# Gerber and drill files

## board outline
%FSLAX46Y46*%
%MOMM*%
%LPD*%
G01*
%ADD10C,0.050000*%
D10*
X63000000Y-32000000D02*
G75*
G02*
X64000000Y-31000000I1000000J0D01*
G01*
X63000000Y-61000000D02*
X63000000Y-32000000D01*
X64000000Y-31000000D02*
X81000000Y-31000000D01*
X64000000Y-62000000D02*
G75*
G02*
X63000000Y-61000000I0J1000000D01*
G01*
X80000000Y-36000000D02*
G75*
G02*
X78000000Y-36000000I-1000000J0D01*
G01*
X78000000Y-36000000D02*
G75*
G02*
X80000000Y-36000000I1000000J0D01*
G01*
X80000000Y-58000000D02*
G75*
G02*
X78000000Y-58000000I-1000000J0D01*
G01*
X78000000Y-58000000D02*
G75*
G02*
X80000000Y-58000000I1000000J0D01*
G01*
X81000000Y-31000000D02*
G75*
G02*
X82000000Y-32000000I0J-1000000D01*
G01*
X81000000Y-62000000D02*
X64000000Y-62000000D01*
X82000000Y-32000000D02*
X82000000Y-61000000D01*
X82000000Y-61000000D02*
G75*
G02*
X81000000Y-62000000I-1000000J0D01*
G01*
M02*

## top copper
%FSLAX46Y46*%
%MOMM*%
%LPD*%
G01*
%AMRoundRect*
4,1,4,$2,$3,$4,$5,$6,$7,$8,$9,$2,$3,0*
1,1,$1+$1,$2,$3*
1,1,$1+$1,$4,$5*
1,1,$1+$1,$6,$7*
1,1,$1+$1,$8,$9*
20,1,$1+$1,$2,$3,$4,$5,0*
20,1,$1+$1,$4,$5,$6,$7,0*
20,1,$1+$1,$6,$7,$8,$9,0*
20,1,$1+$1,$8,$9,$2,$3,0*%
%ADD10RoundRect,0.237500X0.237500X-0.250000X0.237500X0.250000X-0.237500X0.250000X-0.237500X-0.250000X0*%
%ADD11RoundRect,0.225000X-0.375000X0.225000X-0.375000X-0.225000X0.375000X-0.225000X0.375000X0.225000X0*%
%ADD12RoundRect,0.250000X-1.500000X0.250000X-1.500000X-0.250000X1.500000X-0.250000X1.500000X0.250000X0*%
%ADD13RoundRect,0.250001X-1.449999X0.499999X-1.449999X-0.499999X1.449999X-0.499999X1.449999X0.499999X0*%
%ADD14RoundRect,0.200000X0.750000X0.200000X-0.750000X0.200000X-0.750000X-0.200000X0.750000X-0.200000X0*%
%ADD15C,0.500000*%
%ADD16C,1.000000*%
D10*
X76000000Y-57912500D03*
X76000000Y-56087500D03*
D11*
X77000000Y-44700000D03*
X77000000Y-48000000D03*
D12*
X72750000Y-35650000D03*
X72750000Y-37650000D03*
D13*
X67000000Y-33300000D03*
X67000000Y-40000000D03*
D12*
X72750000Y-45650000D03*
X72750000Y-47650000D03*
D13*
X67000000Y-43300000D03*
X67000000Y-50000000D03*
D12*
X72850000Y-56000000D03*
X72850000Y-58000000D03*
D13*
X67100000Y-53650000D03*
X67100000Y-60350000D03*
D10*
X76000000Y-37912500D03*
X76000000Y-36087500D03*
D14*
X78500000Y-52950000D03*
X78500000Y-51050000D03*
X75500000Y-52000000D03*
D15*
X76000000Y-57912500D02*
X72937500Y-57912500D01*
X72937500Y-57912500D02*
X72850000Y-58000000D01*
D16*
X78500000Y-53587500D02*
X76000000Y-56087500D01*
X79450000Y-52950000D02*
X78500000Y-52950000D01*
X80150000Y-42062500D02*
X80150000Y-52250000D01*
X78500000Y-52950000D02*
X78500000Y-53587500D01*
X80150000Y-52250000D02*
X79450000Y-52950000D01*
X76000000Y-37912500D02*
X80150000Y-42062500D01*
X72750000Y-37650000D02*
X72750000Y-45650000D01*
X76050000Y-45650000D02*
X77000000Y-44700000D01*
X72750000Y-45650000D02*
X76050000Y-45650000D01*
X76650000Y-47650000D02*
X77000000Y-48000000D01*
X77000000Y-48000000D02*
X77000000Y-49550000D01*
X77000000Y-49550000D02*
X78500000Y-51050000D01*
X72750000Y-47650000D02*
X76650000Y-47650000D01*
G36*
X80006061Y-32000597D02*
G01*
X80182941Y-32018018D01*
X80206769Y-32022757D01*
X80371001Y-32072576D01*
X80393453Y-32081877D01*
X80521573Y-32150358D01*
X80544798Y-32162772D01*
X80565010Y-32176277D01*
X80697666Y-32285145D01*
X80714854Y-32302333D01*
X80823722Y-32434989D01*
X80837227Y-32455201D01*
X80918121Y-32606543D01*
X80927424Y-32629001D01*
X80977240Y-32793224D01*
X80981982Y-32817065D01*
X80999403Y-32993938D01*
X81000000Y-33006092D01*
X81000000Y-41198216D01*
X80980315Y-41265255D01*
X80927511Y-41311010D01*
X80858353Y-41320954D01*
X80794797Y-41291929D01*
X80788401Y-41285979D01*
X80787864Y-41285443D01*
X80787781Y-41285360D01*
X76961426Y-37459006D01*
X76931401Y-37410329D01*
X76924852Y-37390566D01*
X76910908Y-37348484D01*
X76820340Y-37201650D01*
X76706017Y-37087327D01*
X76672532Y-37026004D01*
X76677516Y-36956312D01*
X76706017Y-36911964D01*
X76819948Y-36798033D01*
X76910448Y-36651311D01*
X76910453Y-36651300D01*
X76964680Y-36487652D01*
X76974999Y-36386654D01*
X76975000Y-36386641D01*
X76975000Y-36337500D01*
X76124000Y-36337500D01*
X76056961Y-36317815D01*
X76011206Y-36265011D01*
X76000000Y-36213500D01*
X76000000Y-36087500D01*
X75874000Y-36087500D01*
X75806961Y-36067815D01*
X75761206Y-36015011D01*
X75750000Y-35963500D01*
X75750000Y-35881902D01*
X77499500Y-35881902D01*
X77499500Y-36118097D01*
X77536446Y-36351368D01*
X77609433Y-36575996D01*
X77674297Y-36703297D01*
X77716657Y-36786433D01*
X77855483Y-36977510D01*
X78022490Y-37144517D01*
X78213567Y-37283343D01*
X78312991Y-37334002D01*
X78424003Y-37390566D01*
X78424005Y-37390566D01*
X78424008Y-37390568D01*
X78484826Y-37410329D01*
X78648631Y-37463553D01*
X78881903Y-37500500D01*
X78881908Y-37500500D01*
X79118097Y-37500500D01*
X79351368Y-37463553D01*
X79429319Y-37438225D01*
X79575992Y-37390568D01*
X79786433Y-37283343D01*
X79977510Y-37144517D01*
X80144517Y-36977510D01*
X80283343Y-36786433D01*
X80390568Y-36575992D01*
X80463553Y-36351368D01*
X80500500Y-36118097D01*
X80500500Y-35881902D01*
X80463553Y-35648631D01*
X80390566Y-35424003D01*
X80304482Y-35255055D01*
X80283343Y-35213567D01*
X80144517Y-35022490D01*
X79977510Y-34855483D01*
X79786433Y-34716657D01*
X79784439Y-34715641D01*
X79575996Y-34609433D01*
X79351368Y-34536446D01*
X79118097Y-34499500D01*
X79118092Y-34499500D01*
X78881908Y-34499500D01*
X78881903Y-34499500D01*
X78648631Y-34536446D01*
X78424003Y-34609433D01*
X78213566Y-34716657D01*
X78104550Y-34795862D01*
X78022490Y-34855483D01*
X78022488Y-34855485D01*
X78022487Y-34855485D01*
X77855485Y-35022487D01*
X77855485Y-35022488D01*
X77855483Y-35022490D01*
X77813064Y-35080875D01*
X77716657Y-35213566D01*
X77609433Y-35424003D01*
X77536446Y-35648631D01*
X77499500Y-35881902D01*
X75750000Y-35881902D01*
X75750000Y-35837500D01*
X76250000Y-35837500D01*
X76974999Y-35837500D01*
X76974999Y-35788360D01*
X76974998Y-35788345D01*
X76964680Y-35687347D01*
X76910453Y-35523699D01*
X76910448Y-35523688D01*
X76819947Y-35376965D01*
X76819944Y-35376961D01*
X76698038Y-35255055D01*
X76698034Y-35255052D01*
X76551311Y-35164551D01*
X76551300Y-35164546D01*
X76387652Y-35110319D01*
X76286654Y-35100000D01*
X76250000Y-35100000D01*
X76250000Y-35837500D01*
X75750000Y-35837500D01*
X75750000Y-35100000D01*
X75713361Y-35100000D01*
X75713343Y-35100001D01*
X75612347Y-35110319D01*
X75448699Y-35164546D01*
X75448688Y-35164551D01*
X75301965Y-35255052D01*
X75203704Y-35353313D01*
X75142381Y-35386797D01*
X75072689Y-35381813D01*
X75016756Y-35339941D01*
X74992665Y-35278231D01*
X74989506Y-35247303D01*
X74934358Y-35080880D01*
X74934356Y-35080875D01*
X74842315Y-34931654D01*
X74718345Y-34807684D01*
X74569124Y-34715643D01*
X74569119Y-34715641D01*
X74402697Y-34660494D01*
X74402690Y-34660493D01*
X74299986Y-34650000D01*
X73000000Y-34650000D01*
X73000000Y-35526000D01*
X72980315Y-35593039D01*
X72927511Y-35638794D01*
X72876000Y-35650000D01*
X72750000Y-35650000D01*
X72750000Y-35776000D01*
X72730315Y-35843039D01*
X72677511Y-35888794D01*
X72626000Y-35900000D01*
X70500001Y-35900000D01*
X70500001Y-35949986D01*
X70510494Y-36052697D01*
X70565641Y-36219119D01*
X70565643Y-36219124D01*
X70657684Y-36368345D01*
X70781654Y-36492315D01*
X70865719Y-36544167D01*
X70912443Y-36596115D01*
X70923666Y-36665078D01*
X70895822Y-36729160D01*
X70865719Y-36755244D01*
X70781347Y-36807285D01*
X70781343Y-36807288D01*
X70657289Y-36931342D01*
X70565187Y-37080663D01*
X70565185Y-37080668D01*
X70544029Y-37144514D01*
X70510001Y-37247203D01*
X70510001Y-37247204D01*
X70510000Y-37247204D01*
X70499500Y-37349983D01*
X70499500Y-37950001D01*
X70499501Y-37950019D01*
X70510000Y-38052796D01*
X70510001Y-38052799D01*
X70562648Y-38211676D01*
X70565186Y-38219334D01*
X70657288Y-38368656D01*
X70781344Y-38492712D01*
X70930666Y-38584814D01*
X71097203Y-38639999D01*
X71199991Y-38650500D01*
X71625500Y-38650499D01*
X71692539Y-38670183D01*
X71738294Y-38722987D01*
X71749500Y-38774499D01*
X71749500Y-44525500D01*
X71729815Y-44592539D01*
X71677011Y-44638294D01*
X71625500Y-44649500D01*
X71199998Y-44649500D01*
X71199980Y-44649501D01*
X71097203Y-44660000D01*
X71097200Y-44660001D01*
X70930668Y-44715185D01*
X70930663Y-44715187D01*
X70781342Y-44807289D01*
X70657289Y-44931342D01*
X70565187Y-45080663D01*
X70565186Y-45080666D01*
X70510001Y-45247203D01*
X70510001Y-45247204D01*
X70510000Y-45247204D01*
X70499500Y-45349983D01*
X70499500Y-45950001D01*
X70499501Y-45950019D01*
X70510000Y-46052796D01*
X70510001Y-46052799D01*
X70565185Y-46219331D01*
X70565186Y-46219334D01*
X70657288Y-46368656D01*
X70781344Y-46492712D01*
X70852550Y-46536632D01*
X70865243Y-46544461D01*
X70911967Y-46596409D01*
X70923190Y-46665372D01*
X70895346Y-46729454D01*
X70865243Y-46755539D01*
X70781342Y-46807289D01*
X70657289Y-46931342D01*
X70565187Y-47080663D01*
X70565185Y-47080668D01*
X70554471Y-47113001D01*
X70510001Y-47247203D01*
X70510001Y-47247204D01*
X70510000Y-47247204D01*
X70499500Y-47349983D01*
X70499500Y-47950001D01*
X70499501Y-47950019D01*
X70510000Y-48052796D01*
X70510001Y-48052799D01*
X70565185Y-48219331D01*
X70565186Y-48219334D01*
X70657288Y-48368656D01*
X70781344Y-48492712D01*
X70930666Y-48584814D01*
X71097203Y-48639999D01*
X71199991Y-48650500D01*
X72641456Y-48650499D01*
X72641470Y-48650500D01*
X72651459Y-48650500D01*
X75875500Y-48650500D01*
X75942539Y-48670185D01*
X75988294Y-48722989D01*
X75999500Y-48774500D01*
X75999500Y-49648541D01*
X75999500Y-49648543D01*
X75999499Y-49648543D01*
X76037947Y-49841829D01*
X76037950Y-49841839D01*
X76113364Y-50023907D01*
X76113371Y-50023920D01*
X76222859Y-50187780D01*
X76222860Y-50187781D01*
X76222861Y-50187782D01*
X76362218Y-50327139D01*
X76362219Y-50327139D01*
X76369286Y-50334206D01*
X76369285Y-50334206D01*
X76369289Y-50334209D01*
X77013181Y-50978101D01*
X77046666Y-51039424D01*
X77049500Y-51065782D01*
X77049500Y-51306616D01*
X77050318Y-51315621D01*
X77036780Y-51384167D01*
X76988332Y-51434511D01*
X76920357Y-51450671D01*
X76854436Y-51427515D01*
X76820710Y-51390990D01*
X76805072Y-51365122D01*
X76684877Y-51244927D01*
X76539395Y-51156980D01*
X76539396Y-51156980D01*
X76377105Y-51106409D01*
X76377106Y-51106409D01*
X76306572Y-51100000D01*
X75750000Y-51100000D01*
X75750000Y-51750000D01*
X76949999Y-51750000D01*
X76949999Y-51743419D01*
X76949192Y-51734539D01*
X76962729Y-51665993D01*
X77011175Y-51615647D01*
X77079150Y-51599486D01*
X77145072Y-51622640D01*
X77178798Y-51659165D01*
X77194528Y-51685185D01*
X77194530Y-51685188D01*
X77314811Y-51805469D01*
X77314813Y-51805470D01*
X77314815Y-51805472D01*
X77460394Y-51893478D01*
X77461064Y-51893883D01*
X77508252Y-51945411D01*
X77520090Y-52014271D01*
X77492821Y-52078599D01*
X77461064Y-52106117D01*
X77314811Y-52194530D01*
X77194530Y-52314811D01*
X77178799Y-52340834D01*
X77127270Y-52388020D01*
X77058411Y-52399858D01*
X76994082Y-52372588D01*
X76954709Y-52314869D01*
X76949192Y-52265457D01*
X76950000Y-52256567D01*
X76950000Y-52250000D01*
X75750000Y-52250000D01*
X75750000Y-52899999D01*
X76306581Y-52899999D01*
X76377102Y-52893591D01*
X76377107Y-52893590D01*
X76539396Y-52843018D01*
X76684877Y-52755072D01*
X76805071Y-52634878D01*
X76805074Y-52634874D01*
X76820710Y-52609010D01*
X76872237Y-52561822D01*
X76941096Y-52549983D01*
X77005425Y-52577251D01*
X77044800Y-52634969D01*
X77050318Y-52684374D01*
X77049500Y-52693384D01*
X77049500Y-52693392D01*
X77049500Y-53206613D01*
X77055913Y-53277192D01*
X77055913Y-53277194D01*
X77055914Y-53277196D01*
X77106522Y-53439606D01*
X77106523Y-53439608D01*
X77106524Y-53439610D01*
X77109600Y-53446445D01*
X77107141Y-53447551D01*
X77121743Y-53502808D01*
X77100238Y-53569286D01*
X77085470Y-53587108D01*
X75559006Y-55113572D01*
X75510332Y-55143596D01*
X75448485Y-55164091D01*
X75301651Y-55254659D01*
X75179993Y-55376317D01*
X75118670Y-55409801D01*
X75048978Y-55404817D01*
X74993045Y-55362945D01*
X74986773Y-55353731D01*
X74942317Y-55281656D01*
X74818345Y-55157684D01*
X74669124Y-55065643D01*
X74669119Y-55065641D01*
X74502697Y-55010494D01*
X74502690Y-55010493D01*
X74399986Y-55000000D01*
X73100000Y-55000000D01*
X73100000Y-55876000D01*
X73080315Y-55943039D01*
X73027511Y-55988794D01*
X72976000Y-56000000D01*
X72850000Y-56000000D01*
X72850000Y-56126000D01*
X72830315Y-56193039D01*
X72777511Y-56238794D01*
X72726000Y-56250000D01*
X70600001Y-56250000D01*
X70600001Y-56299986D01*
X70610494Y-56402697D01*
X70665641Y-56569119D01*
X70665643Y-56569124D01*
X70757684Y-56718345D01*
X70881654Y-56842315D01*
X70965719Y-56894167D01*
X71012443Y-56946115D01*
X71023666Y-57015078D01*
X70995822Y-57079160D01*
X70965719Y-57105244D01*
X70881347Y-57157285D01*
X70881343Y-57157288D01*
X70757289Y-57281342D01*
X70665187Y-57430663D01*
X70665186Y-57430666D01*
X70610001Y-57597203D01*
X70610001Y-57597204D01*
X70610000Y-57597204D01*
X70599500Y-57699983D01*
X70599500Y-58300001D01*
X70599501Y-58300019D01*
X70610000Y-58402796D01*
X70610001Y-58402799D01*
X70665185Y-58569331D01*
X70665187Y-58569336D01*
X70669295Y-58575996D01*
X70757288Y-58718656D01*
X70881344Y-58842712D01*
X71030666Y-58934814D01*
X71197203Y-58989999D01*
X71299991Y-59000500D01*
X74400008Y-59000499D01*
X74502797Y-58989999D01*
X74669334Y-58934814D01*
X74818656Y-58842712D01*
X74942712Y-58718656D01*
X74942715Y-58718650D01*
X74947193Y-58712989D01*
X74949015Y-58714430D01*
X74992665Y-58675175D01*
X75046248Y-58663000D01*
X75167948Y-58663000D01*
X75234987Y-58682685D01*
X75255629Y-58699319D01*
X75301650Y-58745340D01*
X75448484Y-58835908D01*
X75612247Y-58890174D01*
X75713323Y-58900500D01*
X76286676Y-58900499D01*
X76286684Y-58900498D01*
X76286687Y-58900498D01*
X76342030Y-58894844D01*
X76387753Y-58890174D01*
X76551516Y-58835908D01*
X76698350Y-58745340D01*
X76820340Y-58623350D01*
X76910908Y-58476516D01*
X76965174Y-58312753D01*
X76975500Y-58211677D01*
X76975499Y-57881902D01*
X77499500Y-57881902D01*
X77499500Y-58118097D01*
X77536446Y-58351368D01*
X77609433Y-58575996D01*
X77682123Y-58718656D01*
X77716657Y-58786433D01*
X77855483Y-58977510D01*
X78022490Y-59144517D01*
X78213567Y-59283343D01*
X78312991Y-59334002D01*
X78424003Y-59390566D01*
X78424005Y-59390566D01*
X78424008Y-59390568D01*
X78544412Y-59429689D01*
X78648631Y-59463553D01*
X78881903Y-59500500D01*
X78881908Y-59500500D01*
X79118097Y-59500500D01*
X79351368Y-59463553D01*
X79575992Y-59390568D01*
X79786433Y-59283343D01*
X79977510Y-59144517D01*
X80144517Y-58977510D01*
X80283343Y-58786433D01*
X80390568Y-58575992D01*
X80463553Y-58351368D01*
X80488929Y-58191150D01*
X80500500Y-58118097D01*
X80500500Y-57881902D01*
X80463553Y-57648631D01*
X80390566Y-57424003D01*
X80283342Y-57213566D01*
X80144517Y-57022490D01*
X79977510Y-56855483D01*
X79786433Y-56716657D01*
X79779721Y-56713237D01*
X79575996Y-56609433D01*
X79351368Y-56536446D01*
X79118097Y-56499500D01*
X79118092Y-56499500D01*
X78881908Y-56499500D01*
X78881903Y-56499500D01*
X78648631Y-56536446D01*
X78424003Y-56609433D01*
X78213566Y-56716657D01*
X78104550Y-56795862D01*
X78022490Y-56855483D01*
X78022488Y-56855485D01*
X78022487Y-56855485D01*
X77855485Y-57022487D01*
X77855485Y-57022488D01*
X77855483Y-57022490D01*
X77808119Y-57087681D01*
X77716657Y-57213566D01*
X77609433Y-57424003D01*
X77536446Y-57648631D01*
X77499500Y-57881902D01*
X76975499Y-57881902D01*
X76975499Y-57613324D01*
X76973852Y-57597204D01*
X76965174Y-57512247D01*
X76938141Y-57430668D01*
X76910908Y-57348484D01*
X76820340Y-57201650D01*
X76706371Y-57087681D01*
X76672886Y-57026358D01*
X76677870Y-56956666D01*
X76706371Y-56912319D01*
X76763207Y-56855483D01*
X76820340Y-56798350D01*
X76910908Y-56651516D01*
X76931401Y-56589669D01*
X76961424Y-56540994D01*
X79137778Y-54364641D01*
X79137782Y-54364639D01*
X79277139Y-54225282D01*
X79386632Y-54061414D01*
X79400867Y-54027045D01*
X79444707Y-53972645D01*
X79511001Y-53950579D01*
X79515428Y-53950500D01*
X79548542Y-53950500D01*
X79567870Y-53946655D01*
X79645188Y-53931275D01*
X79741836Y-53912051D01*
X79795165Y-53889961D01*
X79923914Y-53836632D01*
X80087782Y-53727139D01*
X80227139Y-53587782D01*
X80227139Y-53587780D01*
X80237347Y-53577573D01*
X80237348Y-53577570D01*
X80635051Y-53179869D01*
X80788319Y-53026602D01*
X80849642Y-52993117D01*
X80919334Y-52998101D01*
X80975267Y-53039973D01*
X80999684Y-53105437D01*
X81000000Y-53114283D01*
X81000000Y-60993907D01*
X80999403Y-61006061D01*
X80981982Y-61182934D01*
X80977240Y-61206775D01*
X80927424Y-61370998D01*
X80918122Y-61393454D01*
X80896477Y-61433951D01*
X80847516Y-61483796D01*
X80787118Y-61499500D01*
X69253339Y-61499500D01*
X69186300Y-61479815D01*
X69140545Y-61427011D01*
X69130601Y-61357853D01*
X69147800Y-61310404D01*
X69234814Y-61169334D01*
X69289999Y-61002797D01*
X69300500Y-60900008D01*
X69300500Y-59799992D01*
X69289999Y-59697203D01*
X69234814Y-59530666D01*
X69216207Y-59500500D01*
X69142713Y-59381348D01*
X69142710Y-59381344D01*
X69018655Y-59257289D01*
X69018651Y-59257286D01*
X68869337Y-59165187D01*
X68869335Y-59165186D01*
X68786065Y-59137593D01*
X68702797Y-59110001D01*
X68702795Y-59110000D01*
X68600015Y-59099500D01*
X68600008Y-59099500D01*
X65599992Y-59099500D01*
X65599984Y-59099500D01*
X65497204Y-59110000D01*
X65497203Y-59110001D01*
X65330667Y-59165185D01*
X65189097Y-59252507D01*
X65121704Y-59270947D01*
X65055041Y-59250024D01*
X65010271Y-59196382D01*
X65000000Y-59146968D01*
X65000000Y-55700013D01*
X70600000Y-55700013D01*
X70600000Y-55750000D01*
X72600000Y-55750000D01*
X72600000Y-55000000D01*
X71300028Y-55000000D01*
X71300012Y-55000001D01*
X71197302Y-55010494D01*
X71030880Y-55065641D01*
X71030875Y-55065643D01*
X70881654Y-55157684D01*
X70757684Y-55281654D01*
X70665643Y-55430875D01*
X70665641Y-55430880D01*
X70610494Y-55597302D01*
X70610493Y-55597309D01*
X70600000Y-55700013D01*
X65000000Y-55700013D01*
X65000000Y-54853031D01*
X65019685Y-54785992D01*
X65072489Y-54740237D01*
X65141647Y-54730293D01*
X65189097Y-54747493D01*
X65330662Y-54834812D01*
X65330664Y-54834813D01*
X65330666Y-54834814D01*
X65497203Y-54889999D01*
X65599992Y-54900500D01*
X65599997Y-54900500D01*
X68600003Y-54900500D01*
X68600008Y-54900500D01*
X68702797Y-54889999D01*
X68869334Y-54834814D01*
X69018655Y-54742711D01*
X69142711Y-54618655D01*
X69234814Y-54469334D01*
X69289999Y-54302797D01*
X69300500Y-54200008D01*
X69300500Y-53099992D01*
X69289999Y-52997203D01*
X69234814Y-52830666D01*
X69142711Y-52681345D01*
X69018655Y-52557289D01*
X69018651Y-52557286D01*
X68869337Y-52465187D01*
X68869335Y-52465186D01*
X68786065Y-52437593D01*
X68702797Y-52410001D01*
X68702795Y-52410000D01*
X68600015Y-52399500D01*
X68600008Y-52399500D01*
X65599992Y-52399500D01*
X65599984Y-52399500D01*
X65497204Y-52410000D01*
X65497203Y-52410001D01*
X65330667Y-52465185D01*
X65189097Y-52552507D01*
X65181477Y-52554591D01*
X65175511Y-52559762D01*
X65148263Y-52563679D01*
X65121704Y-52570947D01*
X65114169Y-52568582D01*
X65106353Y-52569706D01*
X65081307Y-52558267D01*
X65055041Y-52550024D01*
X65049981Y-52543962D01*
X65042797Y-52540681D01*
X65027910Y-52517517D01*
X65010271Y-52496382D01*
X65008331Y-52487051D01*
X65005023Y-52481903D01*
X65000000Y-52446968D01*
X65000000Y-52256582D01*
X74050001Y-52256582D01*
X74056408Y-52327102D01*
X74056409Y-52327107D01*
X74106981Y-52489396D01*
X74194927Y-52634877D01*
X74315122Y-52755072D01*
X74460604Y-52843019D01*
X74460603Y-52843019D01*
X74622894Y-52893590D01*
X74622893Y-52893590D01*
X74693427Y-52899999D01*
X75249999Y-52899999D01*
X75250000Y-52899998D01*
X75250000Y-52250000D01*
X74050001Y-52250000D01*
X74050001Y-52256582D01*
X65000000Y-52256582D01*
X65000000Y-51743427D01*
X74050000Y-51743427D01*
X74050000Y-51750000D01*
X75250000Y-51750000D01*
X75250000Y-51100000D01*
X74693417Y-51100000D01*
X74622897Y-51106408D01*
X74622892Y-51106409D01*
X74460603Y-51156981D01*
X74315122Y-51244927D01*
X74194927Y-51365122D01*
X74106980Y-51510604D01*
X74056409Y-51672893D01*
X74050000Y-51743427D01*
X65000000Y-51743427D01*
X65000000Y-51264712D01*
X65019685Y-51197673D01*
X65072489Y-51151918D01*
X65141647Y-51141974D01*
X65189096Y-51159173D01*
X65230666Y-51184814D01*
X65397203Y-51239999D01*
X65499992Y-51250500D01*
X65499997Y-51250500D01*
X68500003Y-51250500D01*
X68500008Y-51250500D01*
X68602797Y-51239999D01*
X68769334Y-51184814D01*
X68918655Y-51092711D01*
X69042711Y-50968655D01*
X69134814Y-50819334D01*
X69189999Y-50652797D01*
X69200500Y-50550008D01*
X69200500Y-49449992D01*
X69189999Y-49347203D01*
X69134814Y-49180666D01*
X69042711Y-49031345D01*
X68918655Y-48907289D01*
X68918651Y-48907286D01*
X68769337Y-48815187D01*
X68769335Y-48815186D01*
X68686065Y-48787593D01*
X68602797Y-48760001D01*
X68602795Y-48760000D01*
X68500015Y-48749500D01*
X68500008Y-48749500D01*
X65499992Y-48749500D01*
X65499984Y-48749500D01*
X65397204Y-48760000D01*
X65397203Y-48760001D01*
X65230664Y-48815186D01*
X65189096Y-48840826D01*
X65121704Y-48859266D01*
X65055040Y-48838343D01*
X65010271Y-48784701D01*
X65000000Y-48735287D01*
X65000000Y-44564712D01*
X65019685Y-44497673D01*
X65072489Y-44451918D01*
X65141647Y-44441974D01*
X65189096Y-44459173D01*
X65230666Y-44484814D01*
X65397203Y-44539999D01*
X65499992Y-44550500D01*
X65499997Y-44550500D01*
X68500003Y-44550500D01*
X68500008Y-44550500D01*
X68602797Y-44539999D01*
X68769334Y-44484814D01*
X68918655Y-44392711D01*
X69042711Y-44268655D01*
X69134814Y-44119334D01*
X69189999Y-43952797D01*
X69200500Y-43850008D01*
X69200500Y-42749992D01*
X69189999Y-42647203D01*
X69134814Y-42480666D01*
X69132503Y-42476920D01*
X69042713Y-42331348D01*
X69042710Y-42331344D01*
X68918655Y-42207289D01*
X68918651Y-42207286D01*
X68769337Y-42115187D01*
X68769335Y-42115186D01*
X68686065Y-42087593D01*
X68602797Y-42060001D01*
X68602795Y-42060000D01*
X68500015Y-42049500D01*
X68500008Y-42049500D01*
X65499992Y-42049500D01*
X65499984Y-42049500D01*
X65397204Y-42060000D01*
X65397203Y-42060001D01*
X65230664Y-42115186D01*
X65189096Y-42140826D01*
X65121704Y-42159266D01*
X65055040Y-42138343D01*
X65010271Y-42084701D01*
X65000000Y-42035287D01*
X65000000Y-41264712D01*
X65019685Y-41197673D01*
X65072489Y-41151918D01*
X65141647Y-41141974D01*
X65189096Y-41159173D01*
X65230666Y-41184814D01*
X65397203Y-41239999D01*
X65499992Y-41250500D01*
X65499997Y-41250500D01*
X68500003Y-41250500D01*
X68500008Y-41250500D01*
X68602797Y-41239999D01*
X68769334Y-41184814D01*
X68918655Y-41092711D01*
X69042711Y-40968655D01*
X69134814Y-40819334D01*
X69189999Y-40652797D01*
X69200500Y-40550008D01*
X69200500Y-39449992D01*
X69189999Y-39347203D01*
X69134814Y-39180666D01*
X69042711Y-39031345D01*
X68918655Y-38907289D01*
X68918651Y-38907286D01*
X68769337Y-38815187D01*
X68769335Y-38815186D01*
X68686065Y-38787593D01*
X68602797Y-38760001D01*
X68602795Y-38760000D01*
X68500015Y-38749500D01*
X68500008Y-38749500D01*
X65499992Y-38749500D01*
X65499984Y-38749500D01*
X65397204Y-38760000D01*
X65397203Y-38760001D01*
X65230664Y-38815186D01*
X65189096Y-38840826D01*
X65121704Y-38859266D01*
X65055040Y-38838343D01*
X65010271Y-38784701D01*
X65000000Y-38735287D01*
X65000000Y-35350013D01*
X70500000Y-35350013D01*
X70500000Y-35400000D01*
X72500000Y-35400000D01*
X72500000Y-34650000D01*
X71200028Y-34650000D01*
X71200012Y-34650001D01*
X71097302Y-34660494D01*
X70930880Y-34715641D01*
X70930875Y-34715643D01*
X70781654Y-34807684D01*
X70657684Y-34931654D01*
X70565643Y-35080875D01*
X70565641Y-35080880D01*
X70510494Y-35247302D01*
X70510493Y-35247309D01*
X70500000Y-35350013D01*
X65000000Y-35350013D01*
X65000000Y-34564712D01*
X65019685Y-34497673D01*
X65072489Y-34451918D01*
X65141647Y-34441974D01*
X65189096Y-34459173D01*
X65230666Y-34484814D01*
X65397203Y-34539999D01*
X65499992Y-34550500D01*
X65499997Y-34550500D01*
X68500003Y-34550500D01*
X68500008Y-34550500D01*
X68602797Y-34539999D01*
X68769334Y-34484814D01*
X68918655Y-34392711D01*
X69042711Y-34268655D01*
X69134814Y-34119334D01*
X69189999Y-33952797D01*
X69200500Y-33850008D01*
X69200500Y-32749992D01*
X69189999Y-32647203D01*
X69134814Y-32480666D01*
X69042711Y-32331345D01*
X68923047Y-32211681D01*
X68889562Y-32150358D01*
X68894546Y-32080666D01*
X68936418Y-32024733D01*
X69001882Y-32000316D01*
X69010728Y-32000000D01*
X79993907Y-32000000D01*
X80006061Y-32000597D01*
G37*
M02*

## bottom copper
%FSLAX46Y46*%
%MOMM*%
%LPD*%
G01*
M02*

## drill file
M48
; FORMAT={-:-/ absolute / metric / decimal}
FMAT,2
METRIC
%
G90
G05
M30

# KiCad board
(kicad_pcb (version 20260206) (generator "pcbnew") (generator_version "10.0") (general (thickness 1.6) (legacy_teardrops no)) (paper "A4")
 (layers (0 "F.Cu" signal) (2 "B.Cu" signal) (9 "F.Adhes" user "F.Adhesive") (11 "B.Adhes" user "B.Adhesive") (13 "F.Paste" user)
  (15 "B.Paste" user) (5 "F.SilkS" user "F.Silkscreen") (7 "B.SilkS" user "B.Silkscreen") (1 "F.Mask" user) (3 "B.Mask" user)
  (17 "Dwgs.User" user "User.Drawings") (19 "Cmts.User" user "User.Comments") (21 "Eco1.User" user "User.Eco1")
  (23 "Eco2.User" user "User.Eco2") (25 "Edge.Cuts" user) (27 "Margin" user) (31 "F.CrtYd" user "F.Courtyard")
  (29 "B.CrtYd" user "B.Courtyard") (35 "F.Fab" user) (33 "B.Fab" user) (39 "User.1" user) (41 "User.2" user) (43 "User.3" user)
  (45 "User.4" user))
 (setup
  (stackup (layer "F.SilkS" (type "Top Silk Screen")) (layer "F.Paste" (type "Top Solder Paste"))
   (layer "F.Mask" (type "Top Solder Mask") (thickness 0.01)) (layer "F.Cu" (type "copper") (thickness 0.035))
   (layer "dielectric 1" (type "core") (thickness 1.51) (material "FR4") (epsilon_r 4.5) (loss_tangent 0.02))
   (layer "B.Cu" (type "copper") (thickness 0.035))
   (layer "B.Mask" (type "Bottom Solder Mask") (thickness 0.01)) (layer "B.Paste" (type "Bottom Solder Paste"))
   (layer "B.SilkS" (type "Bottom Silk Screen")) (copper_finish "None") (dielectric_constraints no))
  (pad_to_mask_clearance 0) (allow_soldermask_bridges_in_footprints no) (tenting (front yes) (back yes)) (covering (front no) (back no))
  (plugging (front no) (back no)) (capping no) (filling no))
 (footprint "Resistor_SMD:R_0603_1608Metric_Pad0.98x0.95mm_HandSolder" (layer "F.Cu") (at 76 57 90)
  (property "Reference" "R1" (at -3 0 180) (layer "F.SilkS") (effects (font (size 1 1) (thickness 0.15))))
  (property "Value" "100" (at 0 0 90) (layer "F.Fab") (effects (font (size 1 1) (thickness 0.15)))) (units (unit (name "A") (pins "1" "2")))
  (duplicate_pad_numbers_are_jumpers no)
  (pad "1" smd roundrect (at -0.9125 0 90) (size 0.975 0.95) (layers "F.Cu" "F.Mask" "F.Paste") (roundrect_rratio 0.25)
   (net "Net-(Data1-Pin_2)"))
  (pad "2" smd roundrect (at 0.9125 0 90) (size 0.975 0.95) (layers "F.Cu" "F.Mask" "F.Paste") (roundrect_rratio 0.25) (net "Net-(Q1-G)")))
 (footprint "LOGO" (layer "F.Cu") (at 80 44 -90)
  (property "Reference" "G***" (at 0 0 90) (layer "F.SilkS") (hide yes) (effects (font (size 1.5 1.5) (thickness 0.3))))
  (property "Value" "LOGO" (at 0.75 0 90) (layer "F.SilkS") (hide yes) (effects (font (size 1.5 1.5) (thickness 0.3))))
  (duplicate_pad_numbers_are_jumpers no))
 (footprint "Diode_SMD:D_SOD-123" (layer "F.Cu") (at 77 46.35 -90)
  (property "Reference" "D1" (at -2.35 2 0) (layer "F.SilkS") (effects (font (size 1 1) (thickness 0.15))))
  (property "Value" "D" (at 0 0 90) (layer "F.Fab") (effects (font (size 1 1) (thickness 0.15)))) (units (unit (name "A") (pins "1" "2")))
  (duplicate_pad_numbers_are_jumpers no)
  (pad "1" smd roundrect (at -1.65 0 270) (size 0.9 1.2) (layers "F.Cu" "F.Mask" "F.Paste") (roundrect_rratio 0.25) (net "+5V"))
  (pad "2" smd roundrect (at 1.65 0 270) (size 0.9 1.2) (layers "F.Cu" "F.Mask" "F.Paste") (roundrect_rratio 0.25) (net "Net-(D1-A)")))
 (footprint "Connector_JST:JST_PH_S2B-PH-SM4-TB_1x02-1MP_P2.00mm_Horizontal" (layer "F.Cu") (at 69.9 36.65 -90)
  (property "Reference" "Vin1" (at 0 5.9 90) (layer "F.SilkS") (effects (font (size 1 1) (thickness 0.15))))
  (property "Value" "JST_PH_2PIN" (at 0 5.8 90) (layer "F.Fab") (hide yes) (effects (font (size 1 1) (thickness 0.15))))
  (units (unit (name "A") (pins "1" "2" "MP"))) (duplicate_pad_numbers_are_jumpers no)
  (pad "1" smd roundrect (at -1 -2.85 270) (size 1 3.5) (layers "F.Cu" "F.Mask" "F.Paste") (roundrect_rratio 0.25) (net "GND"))
  (pad "2" smd roundrect (at 1 -2.85 270) (size 1 3.5) (layers "F.Cu" "F.Mask" "F.Paste") (roundrect_rratio 0.25) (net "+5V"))
  (pad "MP" smd roundrect (at -3.35 2.9 270) (size 1.5 3.4) (layers "F.Cu" "F.Mask" "F.Paste") (roundrect_rratio 0.166667)
   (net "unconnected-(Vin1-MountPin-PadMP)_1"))
  (pad "MP" smd roundrect (at 3.35 2.9 270) (size 1.5 3.4) (layers "F.Cu" "F.Mask" "F.Paste") (roundrect_rratio 0.166667)
   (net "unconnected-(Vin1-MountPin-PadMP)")))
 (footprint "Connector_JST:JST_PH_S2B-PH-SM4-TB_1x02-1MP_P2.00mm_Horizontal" (layer "F.Cu") (at 69.9 46.65 -90)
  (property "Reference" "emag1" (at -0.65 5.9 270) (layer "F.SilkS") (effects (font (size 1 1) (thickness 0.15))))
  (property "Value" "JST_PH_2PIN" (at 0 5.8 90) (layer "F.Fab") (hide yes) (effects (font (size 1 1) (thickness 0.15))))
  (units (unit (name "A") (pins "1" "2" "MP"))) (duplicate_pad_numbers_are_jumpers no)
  (pad "1" smd roundrect (at -1 -2.85 270) (size 1 3.5) (layers "F.Cu" "F.Mask" "F.Paste") (roundrect_rratio 0.25) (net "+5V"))
  (pad "2" smd roundrect (at 1 -2.85 270) (size 1 3.5) (layers "F.Cu" "F.Mask" "F.Paste") (roundrect_rratio 0.25) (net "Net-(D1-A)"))
  (pad "MP" smd roundrect (at -3.35 2.9 270) (size 1.5 3.4) (layers "F.Cu" "F.Mask" "F.Paste") (roundrect_rratio 0.166667)
   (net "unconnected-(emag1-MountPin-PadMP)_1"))
  (pad "MP" smd roundrect (at 3.35 2.9 270) (size 1.5 3.4) (layers "F.Cu" "F.Mask" "F.Paste") (roundrect_rratio 0.166667)
   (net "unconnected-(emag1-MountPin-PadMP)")))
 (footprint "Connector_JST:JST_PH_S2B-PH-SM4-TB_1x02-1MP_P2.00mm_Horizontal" (layer "F.Cu") (at 70 57 -90)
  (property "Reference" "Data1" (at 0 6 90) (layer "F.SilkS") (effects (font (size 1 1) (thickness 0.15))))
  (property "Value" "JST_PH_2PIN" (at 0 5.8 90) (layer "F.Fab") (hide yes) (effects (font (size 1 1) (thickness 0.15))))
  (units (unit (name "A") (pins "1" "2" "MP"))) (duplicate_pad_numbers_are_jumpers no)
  (pad "1" smd roundrect (at -1 -2.85 270) (size 1 3.5) (layers "F.Cu" "F.Mask" "F.Paste") (roundrect_rratio 0.25) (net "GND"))
  (pad "2" smd roundrect (at 1 -2.85 270) (size 1 3.5) (layers "F.Cu" "F.Mask" "F.Paste") (roundrect_rratio 0.25) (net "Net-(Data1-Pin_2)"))
  (pad "MP" smd roundrect (at -3.35 2.9 270) (size 1.5 3.4) (layers "F.Cu" "F.Mask" "F.Paste") (roundrect_rratio 0.166667)
   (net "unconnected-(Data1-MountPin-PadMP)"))
  (pad "MP" smd roundrect (at 3.35 2.9 270) (size 1.5 3.4) (layers "F.Cu" "F.Mask" "F.Paste") (roundrect_rratio 0.166667)
   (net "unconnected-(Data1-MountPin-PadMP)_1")))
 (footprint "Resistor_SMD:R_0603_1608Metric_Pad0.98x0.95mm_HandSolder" (layer "F.Cu") (at 76 37 90)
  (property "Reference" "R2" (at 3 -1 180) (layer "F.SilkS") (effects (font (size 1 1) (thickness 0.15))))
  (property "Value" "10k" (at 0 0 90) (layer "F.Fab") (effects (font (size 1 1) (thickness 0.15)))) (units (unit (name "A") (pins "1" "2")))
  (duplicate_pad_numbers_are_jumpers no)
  (pad "1" smd roundrect (at -0.9125 0 90) (size 0.975 0.95) (layers "F.Cu" "F.Mask" "F.Paste") (roundrect_rratio 0.25) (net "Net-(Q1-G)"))
  (pad "2" smd roundrect (at 0.9125 0 90) (size 0.975 0.95) (layers "F.Cu" "F.Mask" "F.Paste") (roundrect_rratio 0.25) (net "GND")))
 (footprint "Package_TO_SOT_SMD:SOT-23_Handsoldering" (layer "F.Cu") (at 77 52 180)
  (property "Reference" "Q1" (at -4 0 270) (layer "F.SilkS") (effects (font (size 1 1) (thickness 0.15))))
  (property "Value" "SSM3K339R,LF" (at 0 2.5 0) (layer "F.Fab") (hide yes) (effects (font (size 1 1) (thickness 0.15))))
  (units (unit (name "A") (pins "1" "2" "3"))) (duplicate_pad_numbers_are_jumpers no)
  (pad "1" smd roundrect (at -1.5 -0.95 180) (size 1.9 0.8) (layers "F.Cu" "F.Mask" "F.Paste") (roundrect_rratio 0.25) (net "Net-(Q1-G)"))
  (pad "2" smd roundrect (at -1.5 0.95 180) (size 1.9 0.8) (layers "F.Cu" "F.Mask" "F.Paste") (roundrect_rratio 0.25) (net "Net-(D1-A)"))
  (pad "3" smd roundrect (at 1.5 0 180) (size 1.9 0.8) (layers "F.Cu" "F.Mask" "F.Paste") (roundrect_rratio 0.25) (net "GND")))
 (gr_arc (start 63 32) (mid 63.292893 31.292893) (end 64 31) (stroke (width 0.05) (type default)) (layer "Edge.Cuts"))
 (gr_line (start 63 61) (end 63 32) (stroke (width 0.05) (type default)) (layer "Edge.Cuts"))
 (gr_line (start 64 31) (end 81 31) (stroke (width 0.05) (type default)) (layer "Edge.Cuts"))
 (gr_arc (start 64 62) (mid 63.292893 61.707107) (end 63 61) (stroke (width 0.05) (type default)) (layer "Edge.Cuts"))
 (gr_circle (center 79 36) (end 79 37) (stroke (width 0.05) (type default)) (fill no) (layer "Edge.Cuts"))
 (gr_circle (center 79 58) (end 79 59) (stroke (width 0.05) (type default)) (fill no) (layer "Edge.Cuts"))
 (gr_arc (start 81 31) (mid 81.707107 31.292893) (end 82 32) (stroke (width 0.05) (type default)) (layer "Edge.Cuts"))
 (gr_line (start 81 62) (end 64 62) (stroke (width 0.05) (type default)) (layer "Edge.Cuts"))
 (gr_line (start 82 32) (end 82 61) (stroke (width 0.05) (type default)) (layer "Edge.Cuts"))
 (gr_arc (start 82 61) (mid 81.707107 61.707107) (end 81 62) (stroke (width 0.05) (type default)) (layer "Edge.Cuts"))
 (segment (start 76 57.9125) (end 72.9375 57.9125) (width 0.5) (layer "F.Cu") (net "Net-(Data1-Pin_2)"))
 (segment (start 72.9375 57.9125) (end 72.85 58) (width 0.5) (layer "F.Cu") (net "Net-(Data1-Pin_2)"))
 (segment (start 78.5 53.5875) (end 76 56.0875) (width 1) (layer "F.Cu") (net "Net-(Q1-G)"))
 (segment (start 79.45 52.95) (end 78.5 52.95) (width 1) (layer "F.Cu") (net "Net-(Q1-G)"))
 (segment (start 80.15 42.0625) (end 80.15 52.25) (width 1) (layer "F.Cu") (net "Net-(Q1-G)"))
 (segment (start 78.5 52.95) (end 78.5 53.5875) (width 1) (layer "F.Cu") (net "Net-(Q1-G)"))
 (segment (start 80.15 52.25) (end 79.45 52.95) (width 1) (layer "F.Cu") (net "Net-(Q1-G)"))
 (segment (start 76 37.9125) (end 80.15 42.0625) (width 1) (layer "F.Cu") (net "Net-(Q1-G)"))
 (segment (start 72.75 37.65) (end 72.75 45.65) (width 1) (layer "F.Cu") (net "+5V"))
 (segment (start 76.05 45.65) (end 77 44.7) (width 1) (layer "F.Cu") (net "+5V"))
 (segment (start 72.75 45.65) (end 76.05 45.65) (width 1) (layer "F.Cu") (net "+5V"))
 (segment (start 76.65 47.65) (end 77 48) (width 1) (layer "F.Cu") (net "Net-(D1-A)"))
 (segment (start 77 48) (end 77 49.55) (width 1) (layer "F.Cu") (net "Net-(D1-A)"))
 (segment (start 77 49.55) (end 78.5 51.05) (width 1) (layer "F.Cu") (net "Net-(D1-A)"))
 (segment (start 72.75 47.65) (end 76.65 47.65) (width 1) (layer "F.Cu") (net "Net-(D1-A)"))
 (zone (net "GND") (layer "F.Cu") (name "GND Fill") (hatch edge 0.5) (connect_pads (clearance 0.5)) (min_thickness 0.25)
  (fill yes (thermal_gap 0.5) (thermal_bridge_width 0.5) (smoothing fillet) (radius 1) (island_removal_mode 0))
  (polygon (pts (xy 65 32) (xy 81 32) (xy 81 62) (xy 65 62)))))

